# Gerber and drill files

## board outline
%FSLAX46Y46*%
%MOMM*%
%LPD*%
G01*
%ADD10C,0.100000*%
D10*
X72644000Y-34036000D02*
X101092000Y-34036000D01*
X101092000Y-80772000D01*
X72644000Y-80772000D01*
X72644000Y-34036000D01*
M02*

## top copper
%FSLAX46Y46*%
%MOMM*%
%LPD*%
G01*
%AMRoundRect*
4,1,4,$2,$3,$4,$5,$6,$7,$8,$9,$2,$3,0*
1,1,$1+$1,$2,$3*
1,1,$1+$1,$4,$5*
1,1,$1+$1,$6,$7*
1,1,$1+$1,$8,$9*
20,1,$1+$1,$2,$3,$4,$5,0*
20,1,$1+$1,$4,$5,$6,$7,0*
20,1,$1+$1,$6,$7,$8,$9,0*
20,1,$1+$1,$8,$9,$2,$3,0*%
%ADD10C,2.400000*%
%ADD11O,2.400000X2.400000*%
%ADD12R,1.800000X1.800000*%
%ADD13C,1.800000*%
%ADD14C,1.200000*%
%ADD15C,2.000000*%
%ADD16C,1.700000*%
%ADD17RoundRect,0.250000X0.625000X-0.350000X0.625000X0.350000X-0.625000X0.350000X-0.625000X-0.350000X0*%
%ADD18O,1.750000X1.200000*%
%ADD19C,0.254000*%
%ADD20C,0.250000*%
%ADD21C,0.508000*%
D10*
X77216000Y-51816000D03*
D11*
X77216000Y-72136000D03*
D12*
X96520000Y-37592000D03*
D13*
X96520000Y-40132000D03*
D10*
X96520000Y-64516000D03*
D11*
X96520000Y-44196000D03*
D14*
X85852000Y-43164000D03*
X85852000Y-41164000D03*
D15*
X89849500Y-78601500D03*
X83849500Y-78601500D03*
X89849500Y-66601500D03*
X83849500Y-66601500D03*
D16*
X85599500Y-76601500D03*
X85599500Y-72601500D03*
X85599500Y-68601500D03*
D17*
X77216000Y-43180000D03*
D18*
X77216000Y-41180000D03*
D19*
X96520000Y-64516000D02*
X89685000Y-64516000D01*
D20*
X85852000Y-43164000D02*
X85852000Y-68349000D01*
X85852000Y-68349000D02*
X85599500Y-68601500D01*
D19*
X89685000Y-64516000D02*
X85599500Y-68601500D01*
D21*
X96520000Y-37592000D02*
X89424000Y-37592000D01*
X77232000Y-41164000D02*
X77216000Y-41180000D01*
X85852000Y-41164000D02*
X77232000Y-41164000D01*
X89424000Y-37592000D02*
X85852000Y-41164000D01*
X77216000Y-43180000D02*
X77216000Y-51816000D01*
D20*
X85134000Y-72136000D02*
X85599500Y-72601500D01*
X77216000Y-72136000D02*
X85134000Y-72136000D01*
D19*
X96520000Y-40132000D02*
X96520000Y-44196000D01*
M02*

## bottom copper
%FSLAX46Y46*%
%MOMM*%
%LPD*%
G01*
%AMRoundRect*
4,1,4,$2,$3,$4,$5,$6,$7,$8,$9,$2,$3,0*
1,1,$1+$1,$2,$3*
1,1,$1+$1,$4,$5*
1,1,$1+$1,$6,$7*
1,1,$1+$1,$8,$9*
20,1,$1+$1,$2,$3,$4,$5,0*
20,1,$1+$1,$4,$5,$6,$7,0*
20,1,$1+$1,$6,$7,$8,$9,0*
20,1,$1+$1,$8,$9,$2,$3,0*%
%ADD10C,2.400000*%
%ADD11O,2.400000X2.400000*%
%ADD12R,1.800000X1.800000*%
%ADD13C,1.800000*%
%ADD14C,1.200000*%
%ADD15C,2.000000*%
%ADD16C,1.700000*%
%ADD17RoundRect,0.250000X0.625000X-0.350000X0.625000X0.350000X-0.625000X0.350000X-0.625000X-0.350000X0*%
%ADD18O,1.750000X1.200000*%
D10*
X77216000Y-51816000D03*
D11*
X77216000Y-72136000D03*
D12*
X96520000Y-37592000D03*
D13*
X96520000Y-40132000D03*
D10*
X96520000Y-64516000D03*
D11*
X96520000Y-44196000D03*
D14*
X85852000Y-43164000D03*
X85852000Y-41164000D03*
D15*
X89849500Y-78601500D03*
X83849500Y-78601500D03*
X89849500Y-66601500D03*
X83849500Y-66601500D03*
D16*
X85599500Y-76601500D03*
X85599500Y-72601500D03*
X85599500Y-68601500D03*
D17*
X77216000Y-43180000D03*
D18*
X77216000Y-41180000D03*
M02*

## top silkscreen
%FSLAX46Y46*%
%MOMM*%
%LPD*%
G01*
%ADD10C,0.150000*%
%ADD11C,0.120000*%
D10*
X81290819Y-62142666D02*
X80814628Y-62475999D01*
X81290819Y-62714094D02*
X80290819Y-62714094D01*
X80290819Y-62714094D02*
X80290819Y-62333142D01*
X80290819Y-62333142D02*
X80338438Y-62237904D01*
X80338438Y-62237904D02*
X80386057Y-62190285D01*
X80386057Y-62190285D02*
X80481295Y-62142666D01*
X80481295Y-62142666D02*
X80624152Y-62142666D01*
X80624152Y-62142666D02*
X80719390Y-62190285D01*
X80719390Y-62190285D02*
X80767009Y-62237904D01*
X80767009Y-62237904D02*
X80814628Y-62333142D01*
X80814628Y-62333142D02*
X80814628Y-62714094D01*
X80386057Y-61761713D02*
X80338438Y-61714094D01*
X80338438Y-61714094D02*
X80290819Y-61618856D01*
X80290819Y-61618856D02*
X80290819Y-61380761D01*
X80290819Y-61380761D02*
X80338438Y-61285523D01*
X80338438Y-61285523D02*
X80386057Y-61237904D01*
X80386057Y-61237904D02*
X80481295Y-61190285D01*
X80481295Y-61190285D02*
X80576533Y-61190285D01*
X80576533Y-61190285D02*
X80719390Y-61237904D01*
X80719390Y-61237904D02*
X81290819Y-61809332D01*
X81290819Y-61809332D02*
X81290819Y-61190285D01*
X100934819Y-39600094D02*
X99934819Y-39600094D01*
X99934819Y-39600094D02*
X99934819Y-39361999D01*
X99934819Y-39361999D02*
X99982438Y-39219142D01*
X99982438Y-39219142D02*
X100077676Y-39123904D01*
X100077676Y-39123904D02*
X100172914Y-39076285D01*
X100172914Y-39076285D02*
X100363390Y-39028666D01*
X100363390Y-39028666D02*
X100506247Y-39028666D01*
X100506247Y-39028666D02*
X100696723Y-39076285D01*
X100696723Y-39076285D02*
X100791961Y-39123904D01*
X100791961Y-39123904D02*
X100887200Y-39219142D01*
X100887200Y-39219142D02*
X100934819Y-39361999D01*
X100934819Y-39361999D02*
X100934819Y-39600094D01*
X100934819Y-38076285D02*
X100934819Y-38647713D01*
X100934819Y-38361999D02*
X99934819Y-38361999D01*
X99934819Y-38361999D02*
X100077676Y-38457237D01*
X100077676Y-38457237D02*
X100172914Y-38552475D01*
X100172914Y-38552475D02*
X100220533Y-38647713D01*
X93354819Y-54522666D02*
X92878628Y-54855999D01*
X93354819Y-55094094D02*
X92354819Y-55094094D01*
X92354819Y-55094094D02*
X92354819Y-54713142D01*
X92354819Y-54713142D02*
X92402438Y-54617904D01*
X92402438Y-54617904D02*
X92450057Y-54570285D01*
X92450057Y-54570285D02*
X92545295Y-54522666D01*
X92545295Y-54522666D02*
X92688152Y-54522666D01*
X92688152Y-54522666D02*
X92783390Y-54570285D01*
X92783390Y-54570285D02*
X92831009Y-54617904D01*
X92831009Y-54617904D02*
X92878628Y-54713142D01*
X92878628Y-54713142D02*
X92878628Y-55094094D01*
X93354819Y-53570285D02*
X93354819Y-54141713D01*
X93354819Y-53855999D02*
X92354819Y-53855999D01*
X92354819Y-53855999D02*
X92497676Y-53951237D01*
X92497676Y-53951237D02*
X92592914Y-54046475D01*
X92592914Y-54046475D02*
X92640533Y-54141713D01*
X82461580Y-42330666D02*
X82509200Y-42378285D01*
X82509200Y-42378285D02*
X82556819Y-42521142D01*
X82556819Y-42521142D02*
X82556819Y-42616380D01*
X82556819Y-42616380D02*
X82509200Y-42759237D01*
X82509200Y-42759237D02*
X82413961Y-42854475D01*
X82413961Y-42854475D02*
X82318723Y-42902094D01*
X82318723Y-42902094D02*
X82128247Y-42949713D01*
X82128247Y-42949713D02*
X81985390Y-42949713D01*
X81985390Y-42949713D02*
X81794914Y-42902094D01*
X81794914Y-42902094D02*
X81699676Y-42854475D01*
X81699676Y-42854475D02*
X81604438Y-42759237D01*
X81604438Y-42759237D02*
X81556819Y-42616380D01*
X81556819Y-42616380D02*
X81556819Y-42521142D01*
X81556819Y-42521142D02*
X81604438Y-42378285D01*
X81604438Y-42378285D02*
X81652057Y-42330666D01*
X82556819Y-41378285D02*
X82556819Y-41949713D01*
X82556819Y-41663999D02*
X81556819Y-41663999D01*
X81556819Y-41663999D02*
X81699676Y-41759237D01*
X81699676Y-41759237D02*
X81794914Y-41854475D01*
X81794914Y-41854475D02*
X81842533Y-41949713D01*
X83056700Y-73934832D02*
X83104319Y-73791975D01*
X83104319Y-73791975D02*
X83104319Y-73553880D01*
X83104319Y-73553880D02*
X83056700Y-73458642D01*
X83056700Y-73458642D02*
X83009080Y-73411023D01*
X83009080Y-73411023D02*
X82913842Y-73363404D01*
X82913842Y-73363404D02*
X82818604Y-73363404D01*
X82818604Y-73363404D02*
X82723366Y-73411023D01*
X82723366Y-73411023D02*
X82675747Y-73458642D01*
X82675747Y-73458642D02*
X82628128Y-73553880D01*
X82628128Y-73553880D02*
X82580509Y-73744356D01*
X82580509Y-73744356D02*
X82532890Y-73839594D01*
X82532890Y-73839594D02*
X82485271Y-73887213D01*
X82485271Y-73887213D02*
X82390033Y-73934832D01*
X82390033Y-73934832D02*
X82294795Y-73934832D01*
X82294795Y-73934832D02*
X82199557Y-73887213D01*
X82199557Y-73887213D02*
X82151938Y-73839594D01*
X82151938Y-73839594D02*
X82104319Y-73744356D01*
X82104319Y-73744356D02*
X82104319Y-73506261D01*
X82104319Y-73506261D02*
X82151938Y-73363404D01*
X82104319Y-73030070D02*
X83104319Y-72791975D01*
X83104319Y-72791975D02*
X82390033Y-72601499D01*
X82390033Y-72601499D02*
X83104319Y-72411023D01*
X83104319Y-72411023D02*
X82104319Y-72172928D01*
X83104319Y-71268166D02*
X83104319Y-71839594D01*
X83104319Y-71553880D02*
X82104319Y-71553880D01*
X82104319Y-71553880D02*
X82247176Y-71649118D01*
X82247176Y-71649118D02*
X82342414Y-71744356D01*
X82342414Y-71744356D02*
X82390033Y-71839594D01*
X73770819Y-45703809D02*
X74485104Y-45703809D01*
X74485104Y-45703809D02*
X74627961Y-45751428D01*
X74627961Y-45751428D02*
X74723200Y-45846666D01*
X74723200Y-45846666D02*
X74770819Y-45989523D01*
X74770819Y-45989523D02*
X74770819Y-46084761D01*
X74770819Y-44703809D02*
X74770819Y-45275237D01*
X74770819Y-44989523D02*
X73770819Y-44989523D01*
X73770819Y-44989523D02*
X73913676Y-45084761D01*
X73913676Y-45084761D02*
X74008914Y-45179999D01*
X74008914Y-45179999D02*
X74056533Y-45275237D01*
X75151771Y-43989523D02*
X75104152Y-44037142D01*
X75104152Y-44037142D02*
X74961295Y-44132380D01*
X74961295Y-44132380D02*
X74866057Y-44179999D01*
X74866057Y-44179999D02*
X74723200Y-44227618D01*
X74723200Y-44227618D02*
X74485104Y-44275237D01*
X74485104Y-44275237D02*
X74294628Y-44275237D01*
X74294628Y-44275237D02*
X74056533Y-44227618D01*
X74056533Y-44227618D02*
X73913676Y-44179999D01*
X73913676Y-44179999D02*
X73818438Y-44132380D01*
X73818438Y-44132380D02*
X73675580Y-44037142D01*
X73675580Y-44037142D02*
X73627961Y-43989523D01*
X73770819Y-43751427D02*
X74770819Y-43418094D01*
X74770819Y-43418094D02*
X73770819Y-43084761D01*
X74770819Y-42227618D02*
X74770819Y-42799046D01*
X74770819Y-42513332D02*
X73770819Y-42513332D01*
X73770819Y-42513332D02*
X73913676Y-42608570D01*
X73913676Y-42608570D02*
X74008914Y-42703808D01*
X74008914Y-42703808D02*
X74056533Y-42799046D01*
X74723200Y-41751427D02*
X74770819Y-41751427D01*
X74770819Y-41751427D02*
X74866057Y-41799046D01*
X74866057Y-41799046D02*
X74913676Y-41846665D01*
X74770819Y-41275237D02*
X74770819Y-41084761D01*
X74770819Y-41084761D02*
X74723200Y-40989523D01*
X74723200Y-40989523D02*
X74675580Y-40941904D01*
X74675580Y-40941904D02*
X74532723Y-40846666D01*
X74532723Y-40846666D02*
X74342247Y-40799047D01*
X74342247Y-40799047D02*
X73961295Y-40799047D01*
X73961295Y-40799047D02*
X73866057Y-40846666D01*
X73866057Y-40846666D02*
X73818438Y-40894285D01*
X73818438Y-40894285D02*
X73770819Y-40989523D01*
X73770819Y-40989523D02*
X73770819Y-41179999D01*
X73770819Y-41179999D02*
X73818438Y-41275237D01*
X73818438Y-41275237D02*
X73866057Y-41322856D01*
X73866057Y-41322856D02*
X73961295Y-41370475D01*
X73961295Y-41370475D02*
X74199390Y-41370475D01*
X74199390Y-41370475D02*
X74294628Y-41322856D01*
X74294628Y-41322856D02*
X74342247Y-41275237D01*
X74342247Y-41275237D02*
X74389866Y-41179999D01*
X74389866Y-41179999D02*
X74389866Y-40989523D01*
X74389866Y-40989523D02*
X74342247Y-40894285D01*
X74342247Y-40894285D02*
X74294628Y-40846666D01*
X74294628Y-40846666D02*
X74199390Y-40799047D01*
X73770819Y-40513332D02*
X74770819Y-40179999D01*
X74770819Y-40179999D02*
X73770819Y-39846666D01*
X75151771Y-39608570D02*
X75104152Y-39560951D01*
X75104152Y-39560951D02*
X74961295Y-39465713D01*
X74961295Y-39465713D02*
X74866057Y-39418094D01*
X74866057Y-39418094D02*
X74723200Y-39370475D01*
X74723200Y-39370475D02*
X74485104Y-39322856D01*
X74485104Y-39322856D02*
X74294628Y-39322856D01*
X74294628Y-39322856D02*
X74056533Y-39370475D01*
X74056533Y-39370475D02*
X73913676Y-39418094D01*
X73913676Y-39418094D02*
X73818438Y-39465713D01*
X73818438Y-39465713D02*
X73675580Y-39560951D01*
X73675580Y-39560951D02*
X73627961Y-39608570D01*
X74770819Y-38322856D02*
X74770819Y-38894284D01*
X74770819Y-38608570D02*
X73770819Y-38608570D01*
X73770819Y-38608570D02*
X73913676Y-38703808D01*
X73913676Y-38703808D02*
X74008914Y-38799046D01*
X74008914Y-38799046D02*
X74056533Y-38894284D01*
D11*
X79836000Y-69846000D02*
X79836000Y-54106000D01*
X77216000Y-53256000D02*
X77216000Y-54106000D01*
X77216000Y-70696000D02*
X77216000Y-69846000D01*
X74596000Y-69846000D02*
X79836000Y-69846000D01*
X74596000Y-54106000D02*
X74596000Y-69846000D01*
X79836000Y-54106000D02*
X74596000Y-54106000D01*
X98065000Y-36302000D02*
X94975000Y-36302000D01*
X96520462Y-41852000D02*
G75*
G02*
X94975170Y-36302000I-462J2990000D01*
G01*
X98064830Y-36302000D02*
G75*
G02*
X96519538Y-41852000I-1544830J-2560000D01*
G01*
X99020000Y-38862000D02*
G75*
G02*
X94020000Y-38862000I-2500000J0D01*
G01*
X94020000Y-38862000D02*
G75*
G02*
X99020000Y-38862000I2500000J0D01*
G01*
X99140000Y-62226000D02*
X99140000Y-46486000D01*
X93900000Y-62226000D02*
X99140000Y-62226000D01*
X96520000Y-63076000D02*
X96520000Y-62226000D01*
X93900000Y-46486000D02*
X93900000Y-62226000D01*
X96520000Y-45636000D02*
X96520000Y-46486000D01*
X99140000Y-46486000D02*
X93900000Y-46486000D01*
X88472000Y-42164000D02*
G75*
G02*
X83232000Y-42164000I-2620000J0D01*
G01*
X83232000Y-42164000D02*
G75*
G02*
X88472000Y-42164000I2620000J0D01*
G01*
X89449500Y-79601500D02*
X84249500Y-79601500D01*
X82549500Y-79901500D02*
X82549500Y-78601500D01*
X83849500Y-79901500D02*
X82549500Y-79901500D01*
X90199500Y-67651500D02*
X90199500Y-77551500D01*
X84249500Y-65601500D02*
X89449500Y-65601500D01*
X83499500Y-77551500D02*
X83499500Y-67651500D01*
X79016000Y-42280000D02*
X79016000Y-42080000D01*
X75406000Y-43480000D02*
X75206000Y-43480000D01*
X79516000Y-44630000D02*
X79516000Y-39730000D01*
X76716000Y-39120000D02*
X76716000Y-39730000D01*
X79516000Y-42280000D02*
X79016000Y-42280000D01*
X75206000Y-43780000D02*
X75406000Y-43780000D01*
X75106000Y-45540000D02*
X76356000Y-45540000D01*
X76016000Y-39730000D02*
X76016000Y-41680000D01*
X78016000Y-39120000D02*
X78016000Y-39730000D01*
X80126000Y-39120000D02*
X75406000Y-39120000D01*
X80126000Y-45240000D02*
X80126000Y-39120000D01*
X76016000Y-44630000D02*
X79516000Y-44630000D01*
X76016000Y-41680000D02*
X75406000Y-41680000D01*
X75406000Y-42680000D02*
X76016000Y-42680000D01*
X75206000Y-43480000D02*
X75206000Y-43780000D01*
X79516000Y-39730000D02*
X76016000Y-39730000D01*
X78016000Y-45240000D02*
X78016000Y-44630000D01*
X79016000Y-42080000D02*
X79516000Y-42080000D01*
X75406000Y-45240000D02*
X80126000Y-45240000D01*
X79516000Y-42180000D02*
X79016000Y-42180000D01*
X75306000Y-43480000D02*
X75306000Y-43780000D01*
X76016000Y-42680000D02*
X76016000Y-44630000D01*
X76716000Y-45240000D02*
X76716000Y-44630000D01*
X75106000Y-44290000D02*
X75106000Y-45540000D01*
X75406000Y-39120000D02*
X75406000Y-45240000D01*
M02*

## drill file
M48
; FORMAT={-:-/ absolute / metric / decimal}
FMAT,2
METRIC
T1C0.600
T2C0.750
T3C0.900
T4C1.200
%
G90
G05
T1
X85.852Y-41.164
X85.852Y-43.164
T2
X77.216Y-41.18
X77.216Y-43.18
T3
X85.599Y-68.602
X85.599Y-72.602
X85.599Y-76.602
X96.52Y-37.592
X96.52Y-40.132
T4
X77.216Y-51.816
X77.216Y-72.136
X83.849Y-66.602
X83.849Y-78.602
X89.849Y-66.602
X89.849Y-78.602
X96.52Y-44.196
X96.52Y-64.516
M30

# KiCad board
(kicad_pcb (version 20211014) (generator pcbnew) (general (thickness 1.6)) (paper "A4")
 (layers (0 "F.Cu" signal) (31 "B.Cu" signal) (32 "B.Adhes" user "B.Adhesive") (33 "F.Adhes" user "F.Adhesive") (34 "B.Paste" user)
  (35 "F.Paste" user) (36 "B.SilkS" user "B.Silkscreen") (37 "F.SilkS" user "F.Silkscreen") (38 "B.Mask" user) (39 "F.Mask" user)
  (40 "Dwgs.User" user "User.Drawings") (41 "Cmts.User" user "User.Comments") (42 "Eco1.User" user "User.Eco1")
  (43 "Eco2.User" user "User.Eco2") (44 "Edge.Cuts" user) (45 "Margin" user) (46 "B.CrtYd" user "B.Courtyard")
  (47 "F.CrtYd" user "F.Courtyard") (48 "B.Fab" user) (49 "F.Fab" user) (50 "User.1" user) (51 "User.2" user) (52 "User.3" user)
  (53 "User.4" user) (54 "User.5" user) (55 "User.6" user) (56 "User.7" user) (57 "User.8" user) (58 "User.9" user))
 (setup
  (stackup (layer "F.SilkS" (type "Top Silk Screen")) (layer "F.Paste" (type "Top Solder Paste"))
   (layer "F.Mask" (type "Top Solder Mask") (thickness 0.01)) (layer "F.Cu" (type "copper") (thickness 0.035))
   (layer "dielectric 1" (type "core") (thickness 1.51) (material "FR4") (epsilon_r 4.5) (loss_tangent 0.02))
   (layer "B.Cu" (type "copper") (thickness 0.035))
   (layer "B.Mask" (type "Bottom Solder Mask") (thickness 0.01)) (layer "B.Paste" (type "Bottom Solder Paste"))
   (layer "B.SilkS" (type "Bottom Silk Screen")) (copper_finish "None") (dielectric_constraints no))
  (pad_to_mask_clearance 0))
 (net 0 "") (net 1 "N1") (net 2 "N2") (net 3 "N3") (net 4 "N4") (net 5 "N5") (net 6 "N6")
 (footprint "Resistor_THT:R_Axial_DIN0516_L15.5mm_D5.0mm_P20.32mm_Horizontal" (layer "F.Cu") (at 77.216 51.816 -90)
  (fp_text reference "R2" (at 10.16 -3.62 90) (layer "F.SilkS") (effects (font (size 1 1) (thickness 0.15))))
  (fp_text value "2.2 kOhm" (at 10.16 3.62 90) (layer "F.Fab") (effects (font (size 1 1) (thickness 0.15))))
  (fp_line (start 18.03 -2.62) (end 2.29 -2.62) (layer "F.SilkS") (width 0.12))
  (fp_line (start 1.44 0) (end 2.29 0) (layer "F.SilkS") (width 0.12))
  (fp_line (start 18.88 0) (end 18.03 0) (layer "F.SilkS") (width 0.12))
  (fp_line (start 18.03 2.62) (end 18.03 -2.62) (layer "F.SilkS") (width 0.12))
  (fp_line (start 2.29 2.62) (end 18.03 2.62) (layer "F.SilkS") (width 0.12))
  (fp_line (start 2.29 -2.62) (end 2.29 2.62) (layer "F.SilkS") (width 0.12))
  (pad "1" thru_hole circle (at 0 0 270) (size 2.4 2.4) (drill 1.2) (layers *.Cu *.Mask) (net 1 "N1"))
  (pad "2" thru_hole oval (at 20.32 0 270) (size 2.4 2.4) (drill 1.2) (layers *.Cu *.Mask) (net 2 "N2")))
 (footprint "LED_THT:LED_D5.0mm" (layer "F.Cu") (at 96.52 37.592 -90)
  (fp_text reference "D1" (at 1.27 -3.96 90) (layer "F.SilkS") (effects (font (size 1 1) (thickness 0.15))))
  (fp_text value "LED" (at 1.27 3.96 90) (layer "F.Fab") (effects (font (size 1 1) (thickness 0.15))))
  (fp_line (start -1.29 -1.545) (end -1.29 1.545) (layer "F.SilkS") (width 0.12))
  (fp_arc (start 4.26 -0.000462) (mid 2.072002 2.880433) (end -1.29 1.54483) (layer "F.SilkS") (width 0.12))
  (fp_arc (start -1.29 -1.54483) (mid 2.072002 -2.880433) (end 4.26 0.000462) (layer "F.SilkS") (width 0.12))
  (fp_circle (center 1.27 0) (end 3.77 0) (layer "F.SilkS") (width 0.12) (fill none))
  (pad "1" thru_hole rect (at 0 0 270) (size 1.8 1.8) (drill 0.9) (layers *.Cu *.Mask) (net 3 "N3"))
  (pad "2" thru_hole circle (at 2.54 0 270) (size 1.8 1.8) (drill 0.9) (layers *.Cu *.Mask) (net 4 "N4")))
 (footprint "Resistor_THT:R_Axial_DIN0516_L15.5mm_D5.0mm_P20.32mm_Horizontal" (layer "F.Cu") (at 96.52 64.516 90)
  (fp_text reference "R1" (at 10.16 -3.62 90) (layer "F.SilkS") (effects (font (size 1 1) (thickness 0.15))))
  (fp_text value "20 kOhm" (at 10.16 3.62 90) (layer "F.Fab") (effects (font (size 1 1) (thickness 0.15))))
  (fp_line (start 2.29 2.62) (end 18.03 2.62) (layer "F.SilkS") (width 0.12))
  (fp_line (start 2.29 -2.62) (end 2.29 2.62) (layer "F.SilkS") (width 0.12))
  (fp_line (start 1.44 0) (end 2.29 0) (layer "F.SilkS") (width 0.12))
  (fp_line (start 18.03 -2.62) (end 2.29 -2.62) (layer "F.SilkS") (width 0.12))
  (fp_line (start 18.88 0) (end 18.03 0) (layer "F.SilkS") (width 0.12))
  (fp_line (start 18.03 2.62) (end 18.03 -2.62) (layer "F.SilkS") (width 0.12))
  (pad "1" thru_hole circle (at 0 0 90) (size 2.4 2.4) (drill 1.2) (layers *.Cu *.Mask) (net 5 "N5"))
  (pad "2" thru_hole oval (at 20.32 0 90) (size 2.4 2.4) (drill 1.2) (layers *.Cu *.Mask) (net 4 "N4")))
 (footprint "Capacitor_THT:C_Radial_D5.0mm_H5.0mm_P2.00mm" (layer "F.Cu") (at 85.852 43.164 90)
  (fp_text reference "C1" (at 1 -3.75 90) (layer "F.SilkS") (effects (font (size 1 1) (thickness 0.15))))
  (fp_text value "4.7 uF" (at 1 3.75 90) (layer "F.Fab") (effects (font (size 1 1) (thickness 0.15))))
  (fp_circle (center 1 0) (end 3.62 0) (layer "F.SilkS") (width 0.12) (fill none))
  (pad "1" thru_hole circle (at 0 0 90) (size 1.2 1.2) (drill 0.6) (layers *.Cu *.Mask) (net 5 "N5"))
  (pad "2" thru_hole circle (at 2 0 90) (size 1.2 1.2) (drill 0.6) (layers *.Cu *.Mask) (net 3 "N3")))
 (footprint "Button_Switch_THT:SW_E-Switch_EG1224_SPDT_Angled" (layer "F.Cu") (at 85.5995 76.6015 90)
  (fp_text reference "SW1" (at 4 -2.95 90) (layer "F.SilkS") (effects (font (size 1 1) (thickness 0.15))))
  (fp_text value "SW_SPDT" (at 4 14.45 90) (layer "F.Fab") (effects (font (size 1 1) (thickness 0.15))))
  (fp_line (start -3 3.85) (end -3 -1.35) (layer "F.SilkS") (width 0.12))
  (fp_line (start -3.3 -3.05) (end -2 -3.05) (layer "F.SilkS") (width 0.12))
  (fp_line (start -3.3 -1.75) (end -3.3 -3.05) (layer "F.SilkS") (width 0.12))
  (fp_line (start 8.95 4.6) (end -0.95 4.6) (layer "F.SilkS") (width 0.12))
  (fp_line (start 11 -1.35) (end 11 3.85) (layer "F.SilkS") (width 0.12))
  (fp_line (start -0.95 -2.1) (end 8.95 -2.1) (layer "F.SilkS") (width 0.12))
  (pad "" thru_hole circle (at -2 4.25 90) (size 2 2) (drill 1.2) (layers *.Cu *.Mask))
  (pad "" thru_hole circle (at -2 -1.75 90) (size 2 2) (drill 1.2) (layers *.Cu *.Mask))
  (pad "" thru_hole circle (at 10 4.25 90) (size 2 2) (drill 1.2) (layers *.Cu *.Mask))
  (pad "" thru_hole circle (at 10 -1.75 90) (size 2 2) (drill 1.2) (layers *.Cu *.Mask))
  (pad "1" thru_hole circle (at 0 0 90) (size 1.7 1.7) (drill 0.9) (layers *.Cu *.Mask) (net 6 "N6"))
  (pad "2" thru_hole circle (at 4 0 90) (size 1.7 1.7) (drill 0.9) (layers *.Cu *.Mask) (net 2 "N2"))
  (pad "3" thru_hole circle (at 8 0 90) (size 1.7 1.7) (drill 0.9) (layers *.Cu *.Mask) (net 5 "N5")))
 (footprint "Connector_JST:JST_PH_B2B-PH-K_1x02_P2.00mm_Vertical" (layer "F.Cu") (at 77.216 43.18 90)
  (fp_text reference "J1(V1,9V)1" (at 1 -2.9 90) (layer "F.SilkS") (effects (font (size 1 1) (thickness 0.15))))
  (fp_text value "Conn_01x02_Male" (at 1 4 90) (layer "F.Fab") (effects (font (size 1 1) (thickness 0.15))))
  (fp_line (start 0.9 1.8) (end 1.1 1.8) (layer "F.SilkS") (width 0.12))
  (fp_line (start -0.3 -1.81) (end -0.3 -2.01) (layer "F.SilkS") (width 0.12))
  (fp_line (start -1.45 2.3) (end 3.45 2.3) (layer "F.SilkS") (width 0.12))
  (fp_line (start 4.06 -0.5) (end 3.45 -0.5) (layer "F.SilkS") (width 0.12))
  (fp_line (start 0.9 2.3) (end 0.9 1.8) (layer "F.SilkS") (width 0.12))
  (fp_line (start -0.6 -2.01) (end -0.6 -1.81) (layer "F.SilkS") (width 0.12))
  (fp_line (start -2.36 -2.11) (end -2.36 -0.86) (layer "F.SilkS") (width 0.12))
  (fp_line (start 3.45 -1.2) (end 1.5 -1.2) (layer "F.SilkS") (width 0.12))
  (fp_line (start 4.06 0.8) (end 3.45 0.8) (layer "F.SilkS") (width 0.12))
  (fp_line (start 4.06 2.91) (end 4.06 -1.81) (layer "F.SilkS") (width 0.12))
  (fp_line (start -2.06 2.91) (end 4.06 2.91) (layer "F.SilkS") (width 0.12))
  (fp_line (start -1.45 -1.2) (end -1.45 2.3) (layer "F.SilkS") (width 0.12))
  (fp_line (start 1.5 -1.2) (end 1.5 -1.81) (layer "F.SilkS") (width 0.12))
  (fp_line (start 0.5 -1.81) (end 0.5 -1.2) (layer "F.SilkS") (width 0.12))
  (fp_line (start -0.3 -2.01) (end -0.6 -2.01) (layer "F.SilkS") (width 0.12))
  (fp_line (start 3.45 2.3) (end 3.45 -1.2) (layer "F.SilkS") (width 0.12))
  (fp_line (start -2.06 0.8) (end -1.45 0.8) (layer "F.SilkS") (width 0.12))
  (fp_line (start 1.1 1.8) (end 1.1 2.3) (layer "F.SilkS") (width 0.12))
  (fp_line (start -2.06 -1.81) (end -2.06 2.91) (layer "F.SilkS") (width 0.12))
  (fp_line (start 1 2.3) (end 1 1.8) (layer "F.SilkS") (width 0.12))
  (fp_line (start -0.3 -1.91) (end -0.6 -1.91) (layer "F.SilkS") (width 0.12))
  (fp_line (start 0.5 -1.2) (end -1.45 -1.2) (layer "F.SilkS") (width 0.12))
  (fp_line (start -2.06 -0.5) (end -1.45 -0.5) (layer "F.SilkS") (width 0.12))
  (fp_line (start -1.11 -2.11) (end -2.36 -2.11) (layer "F.SilkS") (width 0.12))
  (fp_line (start 4.06 -1.81) (end -2.06 -1.81) (layer "F.SilkS") (width 0.12))
  (pad "1" thru_hole roundrect (at 0 0 90) (size 1.2 1.75) (drill 0.75) (layers *.Cu *.Mask) (roundrect_rratio 0.208333) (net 1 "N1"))
  (pad "2" thru_hole oval (at 2 0 90) (size 1.2 1.75) (drill 0.75) (layers *.Cu *.Mask) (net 3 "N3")))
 (gr_rect (start 101.092 34.036) (end 72.644 80.772) (layer "Edge.Cuts") (width 0.1) (fill none))
 (segment (start 96.52 64.516) (end 89.685 64.516) (width 0.254) (layer "F.Cu") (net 5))
 (segment (start 85.852 43.164) (end 85.852 68.349) (width 0.25) (layer "F.Cu") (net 5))
 (segment (start 85.852 68.349) (end 85.5995 68.6015) (width 0.25) (layer "F.Cu") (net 5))
 (segment (start 89.685 64.516) (end 85.5995 68.6015) (width 0.254) (layer "F.Cu") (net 5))
 (segment (start 96.52 37.592) (end 89.424 37.592) (width 0.508) (layer "F.Cu") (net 3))
 (segment (start 77.232 41.164) (end 77.216 41.18) (width 0.508) (layer "F.Cu") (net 3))
 (segment (start 85.852 41.164) (end 77.232 41.164) (width 0.508) (layer "F.Cu") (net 3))
 (segment (start 89.424 37.592) (end 85.852 41.164) (width 0.508) (layer "F.Cu") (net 3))
 (segment (start 77.216 43.18) (end 77.216 51.816) (width 0.508) (layer "F.Cu") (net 1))
 (segment (start 85.134 72.136) (end 85.5995 72.6015) (width 0.25) (layer "F.Cu") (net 2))
 (segment (start 77.216 72.136) (end 85.134 72.136) (width 0.25) (layer "F.Cu") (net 2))
 (segment (start 96.52 40.132) (end 96.52 44.196) (width 0.254) (layer "F.Cu") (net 4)))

